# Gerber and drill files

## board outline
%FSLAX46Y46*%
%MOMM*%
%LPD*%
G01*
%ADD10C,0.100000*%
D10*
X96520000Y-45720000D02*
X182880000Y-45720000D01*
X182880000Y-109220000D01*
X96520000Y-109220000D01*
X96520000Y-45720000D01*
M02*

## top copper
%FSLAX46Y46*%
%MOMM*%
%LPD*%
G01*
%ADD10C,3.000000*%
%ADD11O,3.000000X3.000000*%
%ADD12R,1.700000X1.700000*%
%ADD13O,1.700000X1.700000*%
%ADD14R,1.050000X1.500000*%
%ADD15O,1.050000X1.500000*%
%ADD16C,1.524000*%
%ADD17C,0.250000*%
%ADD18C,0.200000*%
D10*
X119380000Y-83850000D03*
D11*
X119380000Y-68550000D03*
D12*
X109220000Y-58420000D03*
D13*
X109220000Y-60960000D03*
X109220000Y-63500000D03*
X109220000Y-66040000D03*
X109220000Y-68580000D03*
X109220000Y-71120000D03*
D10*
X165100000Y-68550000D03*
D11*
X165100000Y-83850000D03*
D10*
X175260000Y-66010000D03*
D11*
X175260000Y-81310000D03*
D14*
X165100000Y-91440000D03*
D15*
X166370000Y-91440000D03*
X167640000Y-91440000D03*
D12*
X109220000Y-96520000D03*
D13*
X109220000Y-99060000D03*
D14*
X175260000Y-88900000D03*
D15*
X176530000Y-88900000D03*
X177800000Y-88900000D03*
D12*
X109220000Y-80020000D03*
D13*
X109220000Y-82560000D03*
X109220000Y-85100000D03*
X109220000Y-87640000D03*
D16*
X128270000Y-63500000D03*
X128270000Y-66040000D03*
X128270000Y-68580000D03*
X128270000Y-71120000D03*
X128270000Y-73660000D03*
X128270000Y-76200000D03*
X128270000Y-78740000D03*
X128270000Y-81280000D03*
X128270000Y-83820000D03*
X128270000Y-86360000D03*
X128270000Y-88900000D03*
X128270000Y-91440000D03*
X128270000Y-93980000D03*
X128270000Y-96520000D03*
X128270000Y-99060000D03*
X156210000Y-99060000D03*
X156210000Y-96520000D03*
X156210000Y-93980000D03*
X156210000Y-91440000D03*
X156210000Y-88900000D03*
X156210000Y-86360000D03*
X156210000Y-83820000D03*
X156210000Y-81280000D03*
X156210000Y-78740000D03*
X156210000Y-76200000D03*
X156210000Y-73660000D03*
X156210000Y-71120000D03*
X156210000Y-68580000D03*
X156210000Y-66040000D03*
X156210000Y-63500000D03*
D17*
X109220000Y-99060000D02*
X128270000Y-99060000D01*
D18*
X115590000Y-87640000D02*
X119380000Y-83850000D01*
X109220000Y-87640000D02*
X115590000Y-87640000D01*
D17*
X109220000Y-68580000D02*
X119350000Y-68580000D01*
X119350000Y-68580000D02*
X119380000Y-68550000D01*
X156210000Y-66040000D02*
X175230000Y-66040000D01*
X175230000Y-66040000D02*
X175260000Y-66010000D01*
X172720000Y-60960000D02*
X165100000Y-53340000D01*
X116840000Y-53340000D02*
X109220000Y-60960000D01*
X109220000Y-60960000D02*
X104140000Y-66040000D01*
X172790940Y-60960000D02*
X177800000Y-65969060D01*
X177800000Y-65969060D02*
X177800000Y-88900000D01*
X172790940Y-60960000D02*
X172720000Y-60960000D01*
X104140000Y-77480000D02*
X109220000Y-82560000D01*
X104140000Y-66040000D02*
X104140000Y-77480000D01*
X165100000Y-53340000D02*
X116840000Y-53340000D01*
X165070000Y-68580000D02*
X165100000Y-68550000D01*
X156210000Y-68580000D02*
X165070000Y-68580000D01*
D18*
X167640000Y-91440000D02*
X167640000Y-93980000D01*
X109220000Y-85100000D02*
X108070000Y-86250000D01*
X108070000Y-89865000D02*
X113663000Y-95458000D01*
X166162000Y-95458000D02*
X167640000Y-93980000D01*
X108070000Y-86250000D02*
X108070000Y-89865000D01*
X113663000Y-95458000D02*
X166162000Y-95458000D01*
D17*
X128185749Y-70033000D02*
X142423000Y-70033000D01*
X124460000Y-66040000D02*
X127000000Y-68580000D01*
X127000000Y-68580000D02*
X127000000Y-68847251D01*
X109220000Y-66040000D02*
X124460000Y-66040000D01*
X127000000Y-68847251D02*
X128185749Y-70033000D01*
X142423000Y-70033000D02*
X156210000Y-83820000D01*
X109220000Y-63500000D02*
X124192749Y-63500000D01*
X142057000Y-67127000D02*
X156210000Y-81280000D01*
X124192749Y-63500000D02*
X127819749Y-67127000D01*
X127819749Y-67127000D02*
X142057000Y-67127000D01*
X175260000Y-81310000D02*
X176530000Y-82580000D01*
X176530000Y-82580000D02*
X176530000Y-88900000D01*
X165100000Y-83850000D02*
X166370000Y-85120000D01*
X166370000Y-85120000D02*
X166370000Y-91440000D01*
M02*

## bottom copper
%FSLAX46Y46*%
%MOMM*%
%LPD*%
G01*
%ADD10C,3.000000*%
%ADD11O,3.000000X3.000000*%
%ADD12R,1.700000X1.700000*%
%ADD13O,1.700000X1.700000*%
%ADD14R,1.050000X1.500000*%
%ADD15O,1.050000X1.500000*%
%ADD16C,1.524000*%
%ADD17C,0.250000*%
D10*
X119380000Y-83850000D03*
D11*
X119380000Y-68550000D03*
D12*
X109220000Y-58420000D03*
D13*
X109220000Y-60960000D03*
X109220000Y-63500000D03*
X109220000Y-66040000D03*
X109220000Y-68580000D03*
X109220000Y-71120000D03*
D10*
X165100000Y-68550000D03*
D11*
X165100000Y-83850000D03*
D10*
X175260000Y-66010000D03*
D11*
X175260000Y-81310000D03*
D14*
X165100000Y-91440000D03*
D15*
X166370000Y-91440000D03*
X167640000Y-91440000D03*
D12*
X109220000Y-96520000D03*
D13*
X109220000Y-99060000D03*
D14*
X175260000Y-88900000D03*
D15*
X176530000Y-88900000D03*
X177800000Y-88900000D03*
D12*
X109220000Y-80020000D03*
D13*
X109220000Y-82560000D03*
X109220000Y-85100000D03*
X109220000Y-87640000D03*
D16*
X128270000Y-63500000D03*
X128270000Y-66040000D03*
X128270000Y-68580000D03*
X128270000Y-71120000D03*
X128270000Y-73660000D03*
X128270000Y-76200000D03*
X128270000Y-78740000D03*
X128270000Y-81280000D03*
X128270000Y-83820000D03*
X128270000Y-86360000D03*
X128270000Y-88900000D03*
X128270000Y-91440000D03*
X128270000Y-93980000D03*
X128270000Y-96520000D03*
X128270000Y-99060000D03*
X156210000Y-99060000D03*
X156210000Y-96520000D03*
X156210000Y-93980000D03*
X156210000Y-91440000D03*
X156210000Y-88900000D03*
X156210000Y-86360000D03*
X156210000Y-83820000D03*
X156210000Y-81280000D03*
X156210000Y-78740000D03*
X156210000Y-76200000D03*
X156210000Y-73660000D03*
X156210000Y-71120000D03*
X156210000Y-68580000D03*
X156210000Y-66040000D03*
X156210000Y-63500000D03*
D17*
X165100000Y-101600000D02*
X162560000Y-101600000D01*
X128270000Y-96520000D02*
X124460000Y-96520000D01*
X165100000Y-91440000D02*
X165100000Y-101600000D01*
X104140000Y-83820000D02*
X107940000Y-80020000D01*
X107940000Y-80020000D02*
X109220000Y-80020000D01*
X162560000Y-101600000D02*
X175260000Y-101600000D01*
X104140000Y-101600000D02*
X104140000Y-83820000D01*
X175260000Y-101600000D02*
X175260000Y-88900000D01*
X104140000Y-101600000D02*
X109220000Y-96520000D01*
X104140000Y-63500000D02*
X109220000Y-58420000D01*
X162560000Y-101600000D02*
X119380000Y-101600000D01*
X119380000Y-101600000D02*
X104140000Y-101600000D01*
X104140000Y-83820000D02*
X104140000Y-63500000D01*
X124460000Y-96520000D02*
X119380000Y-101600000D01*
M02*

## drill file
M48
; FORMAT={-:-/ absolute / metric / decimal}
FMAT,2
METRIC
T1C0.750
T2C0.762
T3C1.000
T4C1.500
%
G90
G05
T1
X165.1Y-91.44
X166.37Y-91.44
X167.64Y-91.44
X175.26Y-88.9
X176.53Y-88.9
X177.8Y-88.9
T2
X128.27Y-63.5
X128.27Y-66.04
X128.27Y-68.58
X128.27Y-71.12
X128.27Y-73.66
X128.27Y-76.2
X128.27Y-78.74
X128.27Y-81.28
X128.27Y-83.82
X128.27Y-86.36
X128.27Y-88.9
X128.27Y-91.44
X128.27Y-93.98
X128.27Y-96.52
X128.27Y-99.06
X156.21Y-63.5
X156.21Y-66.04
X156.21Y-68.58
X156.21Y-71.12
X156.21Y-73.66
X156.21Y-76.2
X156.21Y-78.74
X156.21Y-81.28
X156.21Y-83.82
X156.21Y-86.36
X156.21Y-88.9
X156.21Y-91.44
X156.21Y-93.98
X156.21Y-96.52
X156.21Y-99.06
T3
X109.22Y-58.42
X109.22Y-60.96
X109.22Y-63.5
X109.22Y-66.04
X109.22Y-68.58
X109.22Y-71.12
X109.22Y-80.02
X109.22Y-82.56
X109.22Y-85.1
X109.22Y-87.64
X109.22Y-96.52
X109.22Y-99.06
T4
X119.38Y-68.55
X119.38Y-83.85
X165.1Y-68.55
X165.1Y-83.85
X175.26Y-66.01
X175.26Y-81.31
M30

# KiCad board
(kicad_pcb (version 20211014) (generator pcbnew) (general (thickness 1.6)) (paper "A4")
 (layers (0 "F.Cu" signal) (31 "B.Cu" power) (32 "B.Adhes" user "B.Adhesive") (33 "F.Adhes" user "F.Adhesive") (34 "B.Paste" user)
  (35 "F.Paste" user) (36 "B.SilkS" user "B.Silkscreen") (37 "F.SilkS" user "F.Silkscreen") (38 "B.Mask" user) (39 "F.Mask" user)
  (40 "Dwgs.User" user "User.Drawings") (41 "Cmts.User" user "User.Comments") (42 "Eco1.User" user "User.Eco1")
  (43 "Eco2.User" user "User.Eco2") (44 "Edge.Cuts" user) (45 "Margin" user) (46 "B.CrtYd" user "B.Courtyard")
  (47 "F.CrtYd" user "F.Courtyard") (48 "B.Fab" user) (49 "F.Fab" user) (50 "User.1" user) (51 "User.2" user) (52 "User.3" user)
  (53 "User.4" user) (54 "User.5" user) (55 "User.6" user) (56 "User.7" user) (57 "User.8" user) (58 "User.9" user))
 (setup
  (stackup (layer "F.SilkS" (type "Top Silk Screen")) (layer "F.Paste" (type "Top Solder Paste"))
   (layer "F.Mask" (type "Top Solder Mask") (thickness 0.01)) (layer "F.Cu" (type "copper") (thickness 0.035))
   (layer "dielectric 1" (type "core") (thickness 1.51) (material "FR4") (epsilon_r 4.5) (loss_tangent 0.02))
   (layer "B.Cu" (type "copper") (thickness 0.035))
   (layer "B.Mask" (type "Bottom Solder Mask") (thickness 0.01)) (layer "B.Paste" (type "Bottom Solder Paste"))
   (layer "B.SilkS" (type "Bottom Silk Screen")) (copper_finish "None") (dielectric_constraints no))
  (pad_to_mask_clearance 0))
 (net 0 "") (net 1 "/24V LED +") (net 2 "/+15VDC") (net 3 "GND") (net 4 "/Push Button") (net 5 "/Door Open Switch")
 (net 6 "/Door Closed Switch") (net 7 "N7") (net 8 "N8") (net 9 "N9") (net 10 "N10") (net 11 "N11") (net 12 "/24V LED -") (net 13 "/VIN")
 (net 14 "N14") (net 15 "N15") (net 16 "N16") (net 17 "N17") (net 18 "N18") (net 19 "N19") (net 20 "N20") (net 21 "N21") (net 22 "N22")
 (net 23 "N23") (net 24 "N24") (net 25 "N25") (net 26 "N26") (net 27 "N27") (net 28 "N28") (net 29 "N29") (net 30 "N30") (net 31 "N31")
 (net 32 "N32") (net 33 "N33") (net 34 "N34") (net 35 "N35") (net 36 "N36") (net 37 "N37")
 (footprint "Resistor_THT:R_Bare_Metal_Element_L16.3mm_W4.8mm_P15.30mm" (layer "F.Cu") (at 119.38 83.85 90)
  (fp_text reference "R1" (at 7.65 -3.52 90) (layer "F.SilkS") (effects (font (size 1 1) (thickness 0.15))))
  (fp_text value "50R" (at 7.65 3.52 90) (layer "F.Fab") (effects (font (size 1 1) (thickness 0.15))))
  (pad "1" thru_hole circle (at 0 0 90) (size 3 3) (drill 1.5) (layers *.Cu *.Mask) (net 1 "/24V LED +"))
  (pad "2" thru_hole oval (at 15.3 0 90) (size 3 3) (drill 1.5) (layers *.Cu *.Mask) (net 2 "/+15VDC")))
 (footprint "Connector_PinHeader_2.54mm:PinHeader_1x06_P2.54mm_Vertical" (layer "F.Cu") (at 109.22 58.42)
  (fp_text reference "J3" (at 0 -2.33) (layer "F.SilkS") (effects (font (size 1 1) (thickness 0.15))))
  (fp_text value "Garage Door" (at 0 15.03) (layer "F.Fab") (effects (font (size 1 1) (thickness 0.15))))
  (pad "1" thru_hole rect (at 0 0) (size 1.7 1.7) (drill 1) (layers *.Cu *.Mask) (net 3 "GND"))
  (pad "2" thru_hole oval (at 0 2.54) (size 1.7 1.7) (drill 1) (layers *.Cu *.Mask) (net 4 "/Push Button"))
  (pad "3" thru_hole oval (at 0 5.08) (size 1.7 1.7) (drill 1) (layers *.Cu *.Mask) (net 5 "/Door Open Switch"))
  (pad "4" thru_hole oval (at 0 7.62) (size 1.7 1.7) (drill 1) (layers *.Cu *.Mask) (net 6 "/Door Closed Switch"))
  (pad "5" thru_hole oval (at 0 10.16) (size 1.7 1.7) (drill 1) (layers *.Cu *.Mask) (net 2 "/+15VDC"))
  (pad "6" thru_hole oval (at 0 12.7) (size 1.7 1.7) (drill 1) (layers *.Cu *.Mask) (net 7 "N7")))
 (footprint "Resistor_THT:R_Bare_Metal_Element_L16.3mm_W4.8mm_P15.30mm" (layer "F.Cu") (at 165.1 68.55 -90)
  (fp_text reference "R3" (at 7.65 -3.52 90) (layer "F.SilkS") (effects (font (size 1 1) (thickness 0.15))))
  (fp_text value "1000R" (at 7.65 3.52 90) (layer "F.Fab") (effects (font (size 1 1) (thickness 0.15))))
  (pad "1" thru_hole circle (at 0 0 270) (size 3 3) (drill 1.5) (layers *.Cu *.Mask) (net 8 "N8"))
  (pad "2" thru_hole oval (at 15.3 0 270) (size 3 3) (drill 1.5) (layers *.Cu *.Mask) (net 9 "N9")))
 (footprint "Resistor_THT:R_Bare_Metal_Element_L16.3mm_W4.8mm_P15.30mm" (layer "F.Cu") (at 175.26 66.01 -90)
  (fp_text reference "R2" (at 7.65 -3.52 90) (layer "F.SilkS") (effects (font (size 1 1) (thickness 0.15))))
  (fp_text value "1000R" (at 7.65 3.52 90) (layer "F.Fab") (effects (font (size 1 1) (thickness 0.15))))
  (pad "1" thru_hole circle (at 0 0 270) (size 3 3) (drill 1.5) (layers *.Cu *.Mask) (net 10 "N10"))
  (pad "2" thru_hole oval (at 15.3 0 270) (size 3 3) (drill 1.5) (layers *.Cu *.Mask) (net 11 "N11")))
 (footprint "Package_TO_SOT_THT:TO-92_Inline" (layer "F.Cu") (at 165.1 91.44)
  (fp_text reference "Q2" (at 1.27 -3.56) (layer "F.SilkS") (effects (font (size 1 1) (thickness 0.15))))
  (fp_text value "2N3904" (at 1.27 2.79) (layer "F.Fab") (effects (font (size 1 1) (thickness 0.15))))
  (pad "1" thru_hole rect (at 0 0) (size 1.05 1.5) (drill 0.75) (layers *.Cu *.Mask) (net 3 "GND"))
  (pad "2" thru_hole oval (at 1.27 0) (size 1.05 1.5) (drill 0.75) (layers *.Cu *.Mask) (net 9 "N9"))
  (pad "3" thru_hole oval (at 2.54 0) (size 1.05 1.5) (drill 0.75) (layers *.Cu *.Mask) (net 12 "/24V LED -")))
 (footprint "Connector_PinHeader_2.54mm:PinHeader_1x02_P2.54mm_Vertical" (layer "F.Cu") (at 109.22 96.52)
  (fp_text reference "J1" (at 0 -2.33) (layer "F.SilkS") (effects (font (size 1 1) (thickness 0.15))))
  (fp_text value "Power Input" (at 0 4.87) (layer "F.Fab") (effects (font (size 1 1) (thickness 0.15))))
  (pad "1" thru_hole rect (at 0 0) (size 1.7 1.7) (drill 1) (layers *.Cu *.Mask) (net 3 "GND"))
  (pad "2" thru_hole oval (at 0 2.54) (size 1.7 1.7) (drill 1) (layers *.Cu *.Mask) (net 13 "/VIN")))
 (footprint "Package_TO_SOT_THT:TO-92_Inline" (layer "F.Cu") (at 175.26 88.9)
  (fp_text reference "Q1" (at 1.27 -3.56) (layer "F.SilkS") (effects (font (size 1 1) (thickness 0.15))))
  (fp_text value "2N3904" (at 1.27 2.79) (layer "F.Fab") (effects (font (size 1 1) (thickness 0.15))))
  (pad "1" thru_hole rect (at 0 0) (size 1.05 1.5) (drill 0.75) (layers *.Cu *.Mask) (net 3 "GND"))
  (pad "2" thru_hole oval (at 1.27 0) (size 1.05 1.5) (drill 0.75) (layers *.Cu *.Mask) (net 11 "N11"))
  (pad "3" thru_hole oval (at 2.54 0) (size 1.05 1.5) (drill 0.75) (layers *.Cu *.Mask) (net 4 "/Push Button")))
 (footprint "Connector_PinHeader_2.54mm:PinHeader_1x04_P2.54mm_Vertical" (layer "F.Cu") (at 109.22 80.02)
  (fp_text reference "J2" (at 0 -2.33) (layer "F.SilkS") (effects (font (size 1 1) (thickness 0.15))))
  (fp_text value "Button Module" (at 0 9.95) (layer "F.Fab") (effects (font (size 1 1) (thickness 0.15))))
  (pad "1" thru_hole rect (at 0 0) (size 1.7 1.7) (drill 1) (layers *.Cu *.Mask) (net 3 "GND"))
  (pad "2" thru_hole oval (at 0 2.54) (size 1.7 1.7) (drill 1) (layers *.Cu *.Mask) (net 4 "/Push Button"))
  (pad "3" thru_hole oval (at 0 5.08) (size 1.7 1.7) (drill 1) (layers *.Cu *.Mask) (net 12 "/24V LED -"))
  (pad "4" thru_hole oval (at 0 7.62) (size 1.7 1.7) (drill 1) (layers *.Cu *.Mask) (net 1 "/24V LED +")))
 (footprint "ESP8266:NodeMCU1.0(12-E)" (layer "F.Cu") (at 142.24 81.28)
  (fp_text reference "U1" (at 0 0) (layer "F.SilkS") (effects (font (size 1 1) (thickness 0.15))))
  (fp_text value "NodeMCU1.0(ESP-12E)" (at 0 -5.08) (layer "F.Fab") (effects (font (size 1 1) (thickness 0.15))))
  (pad "1" thru_hole circle locked (at -13.97 -17.78) (size 1.524 1.524) (drill 0.762) (layers *.Cu *.Mask "F.SilkS") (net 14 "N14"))
  (pad "2" thru_hole circle locked (at -13.97 -15.24) (size 1.524 1.524) (drill 0.762) (layers *.Cu *.Mask "F.SilkS") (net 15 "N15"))
  (pad "3" thru_hole circle locked (at -13.97 -12.7) (size 1.524 1.524) (drill 0.762) (layers *.Cu *.Mask "F.SilkS") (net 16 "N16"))
  (pad "4" thru_hole circle locked (at -13.97 -10.16) (size 1.524 1.524) (drill 0.762) (layers *.Cu *.Mask "F.SilkS") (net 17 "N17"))
  (pad "5" thru_hole circle locked (at -13.97 -7.62) (size 1.524 1.524) (drill 0.762) (layers *.Cu *.Mask "F.SilkS") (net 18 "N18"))
  (pad "6" thru_hole circle locked (at -13.97 -5.08) (size 1.524 1.524) (drill 0.762) (layers *.Cu *.Mask "F.SilkS") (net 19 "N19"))
  (pad "7" thru_hole circle locked (at -13.97 -2.54) (size 1.524 1.524) (drill 0.762) (layers *.Cu *.Mask "F.SilkS") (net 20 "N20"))
  (pad "8" thru_hole circle locked (at -13.97 0) (size 1.524 1.524) (drill 0.762) (layers *.Cu *.Mask "F.SilkS") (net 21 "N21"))
  (pad "9" thru_hole circle locked (at -13.97 2.54) (size 1.524 1.524) (drill 0.762) (layers *.Cu *.Mask "F.SilkS") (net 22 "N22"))
  (pad "10" thru_hole circle locked (at -13.97 5.08) (size 1.524 1.524) (drill 0.762) (layers *.Cu *.Mask "F.SilkS") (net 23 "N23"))
  (pad "11" thru_hole circle locked (at -13.97 7.62) (size 1.524 1.524) (drill 0.762) (layers *.Cu *.Mask "F.SilkS") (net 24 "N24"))
  (pad "12" thru_hole circle locked (at -13.97 10.16) (size 1.524 1.524) (drill 0.762) (layers *.Cu *.Mask "F.SilkS") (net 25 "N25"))
  (pad "13" thru_hole circle locked (at -13.97 12.7) (size 1.524 1.524) (drill 0.762) (layers *.Cu *.Mask "F.SilkS") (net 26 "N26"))
  (pad "14" thru_hole circle locked (at -13.97 15.24) (size 1.524 1.524) (drill 0.762) (layers *.Cu *.Mask "F.SilkS") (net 3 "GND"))
  (pad "15" thru_hole circle locked (at -13.97 17.78) (size 1.524 1.524) (drill 0.762) (layers *.Cu *.Mask "F.SilkS") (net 13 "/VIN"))
  (pad "16" thru_hole circle locked (at 13.97 17.78) (size 1.524 1.524) (drill 0.762) (layers *.Cu *.Mask "F.SilkS") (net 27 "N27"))
  (pad "17" thru_hole circle locked (at 13.97 15.24) (size 1.524 1.524) (drill 0.762) (layers *.Cu *.Mask "F.SilkS") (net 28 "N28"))
  (pad "18" thru_hole circle locked (at 13.97 12.7) (size 1.524 1.524) (drill 0.762) (layers *.Cu *.Mask "F.SilkS") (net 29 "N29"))
  (pad "19" thru_hole circle locked (at 13.97 10.16) (size 1.524 1.524) (drill 0.762) (layers *.Cu *.Mask "F.SilkS") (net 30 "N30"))
  (pad "20" thru_hole circle locked (at 13.97 7.62) (size 1.524 1.524) (drill 0.762) (layers *.Cu *.Mask "F.SilkS") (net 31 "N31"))
  (pad "21" thru_hole circle locked (at 13.97 5.08) (size 1.524 1.524) (drill 0.762) (layers *.Cu *.Mask "F.SilkS") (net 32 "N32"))
  (pad "22" thru_hole circle locked (at 13.97 2.54) (size 1.524 1.524) (drill 0.762) (layers *.Cu *.Mask "F.SilkS")
   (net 6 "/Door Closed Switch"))
  (pad "23" thru_hole circle locked (at 13.97 0) (size 1.524 1.524) (drill 0.762) (layers *.Cu *.Mask "F.SilkS") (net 5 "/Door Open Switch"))
  (pad "24" thru_hole circle locked (at 13.97 -2.54) (size 1.524 1.524) (drill 0.762) (layers *.Cu *.Mask "F.SilkS") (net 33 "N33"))
  (pad "25" thru_hole circle locked (at 13.97 -5.08) (size 1.524 1.524) (drill 0.762) (layers *.Cu *.Mask "F.SilkS") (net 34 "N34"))
  (pad "26" thru_hole circle locked (at 13.97 -7.62) (size 1.524 1.524) (drill 0.762) (layers *.Cu *.Mask "F.SilkS") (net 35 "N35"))
  (pad "27" thru_hole circle locked (at 13.97 -10.16) (size 1.524 1.524) (drill 0.762) (layers *.Cu *.Mask "F.SilkS") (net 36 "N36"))
  (pad "28" thru_hole circle locked (at 13.97 -12.7) (size 1.524 1.524) (drill 0.762) (layers *.Cu *.Mask "F.SilkS") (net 8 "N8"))
  (pad "29" thru_hole circle locked (at 13.97 -15.24) (size 1.524 1.524) (drill 0.762) (layers *.Cu *.Mask "F.SilkS") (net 10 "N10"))
  (pad "30" thru_hole circle locked (at 13.97 -17.78) (size 1.524 1.524) (drill 0.762) (layers *.Cu *.Mask "F.SilkS") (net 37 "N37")))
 (gr_rect (start 96.52 45.72) (end 182.88 109.22) (layer "Edge.Cuts") (width 0.1) (fill none))
 (segment (start 109.22 99.06) (end 128.27 99.06) (width 0.25) (layer "F.Cu") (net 13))
 (segment (start 165.1 101.6) (end 162.56 101.6) (width 0.25) (layer "B.Cu") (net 3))
 (segment (start 128.27 96.52) (end 124.46 96.52) (width 0.25) (layer "B.Cu") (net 3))
 (segment (start 165.1 91.44) (end 165.1 101.6) (width 0.25) (layer "B.Cu") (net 3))
 (segment (start 104.14 83.82) (end 107.94 80.02) (width 0.25) (layer "B.Cu") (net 3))
 (segment (start 107.94 80.02) (end 109.22 80.02) (width 0.25) (layer "B.Cu") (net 3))
 (segment (start 162.56 101.6) (end 175.26 101.6) (width 0.25) (layer "B.Cu") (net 3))
 (segment (start 104.14 101.6) (end 104.14 83.82) (width 0.25) (layer "B.Cu") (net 3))
 (segment (start 175.26 101.6) (end 175.26 88.9) (width 0.25) (layer "B.Cu") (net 3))
 (segment (start 104.14 101.6) (end 109.22 96.52) (width 0.25) (layer "B.Cu") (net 3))
 (segment (start 104.14 63.5) (end 109.22 58.42) (width 0.25) (layer "B.Cu") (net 3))
 (segment (start 162.56 101.6) (end 119.38 101.6) (width 0.25) (layer "B.Cu") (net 3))
 (segment (start 119.38 101.6) (end 104.14 101.6) (width 0.25) (layer "B.Cu") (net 3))
 (segment (start 104.14 83.82) (end 104.14 63.5) (width 0.25) (layer "B.Cu") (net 3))
 (segment (start 124.46 96.52) (end 119.38 101.6) (width 0.25) (layer "B.Cu") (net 3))
 (segment (start 115.59 87.64) (end 119.38 83.85) (width 0.2) (layer "F.Cu") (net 1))
 (segment (start 109.22 87.64) (end 115.59 87.64) (width 0.2) (layer "F.Cu") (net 1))
 (segment (start 109.22 68.58) (end 119.35 68.58) (width 0.25) (layer "F.Cu") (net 2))
 (segment (start 119.35 68.58) (end 119.38 68.55) (width 0.25) (layer "F.Cu") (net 2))
 (segment (start 156.21 66.04) (end 175.23 66.04) (width 0.25) (layer "F.Cu") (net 10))
 (segment (start 175.23 66.04) (end 175.26 66.01) (width 0.25) (layer "F.Cu") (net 10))
 (segment (start 172.72 60.96) (end 165.1 53.34) (width 0.25) (layer "F.Cu") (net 4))
 (segment (start 116.84 53.34) (end 109.22 60.96) (width 0.25) (layer "F.Cu") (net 4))
 (segment (start 109.22 60.96) (end 104.14 66.04) (width 0.25) (layer "F.Cu") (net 4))
 (segment (start 172.79094 60.96) (end 177.8 65.96906) (width 0.25) (layer "F.Cu") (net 4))
 (segment (start 177.8 65.96906) (end 177.8 88.9) (width 0.25) (layer "F.Cu") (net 4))
 (segment (start 172.79094 60.96) (end 172.72 60.96) (width 0.25) (layer "F.Cu") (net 4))
 (segment (start 104.14 77.48) (end 109.22 82.56) (width 0.25) (layer "F.Cu") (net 4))
 (segment (start 104.14 66.04) (end 104.14 77.48) (width 0.25) (layer "F.Cu") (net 4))
 (segment (start 165.1 53.34) (end 116.84 53.34) (width 0.25) (layer "F.Cu") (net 4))
 (segment (start 165.07 68.58) (end 165.1 68.55) (width 0.25) (layer "F.Cu") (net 8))
 (segment (start 156.21 68.58) (end 165.07 68.58) (width 0.25) (layer "F.Cu") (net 8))
 (segment (start 167.64 91.44) (end 167.64 93.98) (width 0.2) (layer "F.Cu") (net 12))
 (segment (start 109.22 85.1) (end 108.07 86.25) (width 0.2) (layer "F.Cu") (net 12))
 (segment (start 108.07 89.865) (end 113.663 95.458) (width 0.2) (layer "F.Cu") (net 12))
 (segment (start 166.162 95.458) (end 167.64 93.98) (width 0.2) (layer "F.Cu") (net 12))
 (segment (start 108.07 86.25) (end 108.07 89.865) (width 0.2) (layer "F.Cu") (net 12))
 (segment (start 113.663 95.458) (end 166.162 95.458) (width 0.2) (layer "F.Cu") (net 12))
 (segment (start 128.185749 70.033) (end 142.423 70.033) (width 0.25) (layer "F.Cu") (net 6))
 (segment (start 124.46 66.04) (end 127 68.58) (width 0.25) (layer "F.Cu") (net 6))
 (segment (start 127 68.58) (end 127 68.847251) (width 0.25) (layer "F.Cu") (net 6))
 (segment (start 109.22 66.04) (end 124.46 66.04) (width 0.25) (layer "F.Cu") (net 6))
 (segment (start 127 68.847251) (end 128.185749 70.033) (width 0.25) (layer "F.Cu") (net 6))
 (segment (start 142.423 70.033) (end 156.21 83.82) (width 0.25) (layer "F.Cu") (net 6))
 (segment (start 109.22 63.5) (end 124.192749 63.5) (width 0.25) (layer "F.Cu") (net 5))
 (segment (start 142.057 67.127) (end 156.21 81.28) (width 0.25) (layer "F.Cu") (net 5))
 (segment (start 124.192749 63.5) (end 127.819749 67.127) (width 0.25) (layer "F.Cu") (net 5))
 (segment (start 127.819749 67.127) (end 142.057 67.127) (width 0.25) (layer "F.Cu") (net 5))
 (segment (start 175.26 81.31) (end 176.53 82.58) (width 0.25) (layer "F.Cu") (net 11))
 (segment (start 176.53 82.58) (end 176.53 88.9) (width 0.25) (layer "F.Cu") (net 11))
 (segment (start 165.1 83.85) (end 166.37 85.12) (width 0.25) (layer "F.Cu") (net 9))
 (segment (start 166.37 85.12) (end 166.37 91.44) (width 0.25) (layer "F.Cu") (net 9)))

